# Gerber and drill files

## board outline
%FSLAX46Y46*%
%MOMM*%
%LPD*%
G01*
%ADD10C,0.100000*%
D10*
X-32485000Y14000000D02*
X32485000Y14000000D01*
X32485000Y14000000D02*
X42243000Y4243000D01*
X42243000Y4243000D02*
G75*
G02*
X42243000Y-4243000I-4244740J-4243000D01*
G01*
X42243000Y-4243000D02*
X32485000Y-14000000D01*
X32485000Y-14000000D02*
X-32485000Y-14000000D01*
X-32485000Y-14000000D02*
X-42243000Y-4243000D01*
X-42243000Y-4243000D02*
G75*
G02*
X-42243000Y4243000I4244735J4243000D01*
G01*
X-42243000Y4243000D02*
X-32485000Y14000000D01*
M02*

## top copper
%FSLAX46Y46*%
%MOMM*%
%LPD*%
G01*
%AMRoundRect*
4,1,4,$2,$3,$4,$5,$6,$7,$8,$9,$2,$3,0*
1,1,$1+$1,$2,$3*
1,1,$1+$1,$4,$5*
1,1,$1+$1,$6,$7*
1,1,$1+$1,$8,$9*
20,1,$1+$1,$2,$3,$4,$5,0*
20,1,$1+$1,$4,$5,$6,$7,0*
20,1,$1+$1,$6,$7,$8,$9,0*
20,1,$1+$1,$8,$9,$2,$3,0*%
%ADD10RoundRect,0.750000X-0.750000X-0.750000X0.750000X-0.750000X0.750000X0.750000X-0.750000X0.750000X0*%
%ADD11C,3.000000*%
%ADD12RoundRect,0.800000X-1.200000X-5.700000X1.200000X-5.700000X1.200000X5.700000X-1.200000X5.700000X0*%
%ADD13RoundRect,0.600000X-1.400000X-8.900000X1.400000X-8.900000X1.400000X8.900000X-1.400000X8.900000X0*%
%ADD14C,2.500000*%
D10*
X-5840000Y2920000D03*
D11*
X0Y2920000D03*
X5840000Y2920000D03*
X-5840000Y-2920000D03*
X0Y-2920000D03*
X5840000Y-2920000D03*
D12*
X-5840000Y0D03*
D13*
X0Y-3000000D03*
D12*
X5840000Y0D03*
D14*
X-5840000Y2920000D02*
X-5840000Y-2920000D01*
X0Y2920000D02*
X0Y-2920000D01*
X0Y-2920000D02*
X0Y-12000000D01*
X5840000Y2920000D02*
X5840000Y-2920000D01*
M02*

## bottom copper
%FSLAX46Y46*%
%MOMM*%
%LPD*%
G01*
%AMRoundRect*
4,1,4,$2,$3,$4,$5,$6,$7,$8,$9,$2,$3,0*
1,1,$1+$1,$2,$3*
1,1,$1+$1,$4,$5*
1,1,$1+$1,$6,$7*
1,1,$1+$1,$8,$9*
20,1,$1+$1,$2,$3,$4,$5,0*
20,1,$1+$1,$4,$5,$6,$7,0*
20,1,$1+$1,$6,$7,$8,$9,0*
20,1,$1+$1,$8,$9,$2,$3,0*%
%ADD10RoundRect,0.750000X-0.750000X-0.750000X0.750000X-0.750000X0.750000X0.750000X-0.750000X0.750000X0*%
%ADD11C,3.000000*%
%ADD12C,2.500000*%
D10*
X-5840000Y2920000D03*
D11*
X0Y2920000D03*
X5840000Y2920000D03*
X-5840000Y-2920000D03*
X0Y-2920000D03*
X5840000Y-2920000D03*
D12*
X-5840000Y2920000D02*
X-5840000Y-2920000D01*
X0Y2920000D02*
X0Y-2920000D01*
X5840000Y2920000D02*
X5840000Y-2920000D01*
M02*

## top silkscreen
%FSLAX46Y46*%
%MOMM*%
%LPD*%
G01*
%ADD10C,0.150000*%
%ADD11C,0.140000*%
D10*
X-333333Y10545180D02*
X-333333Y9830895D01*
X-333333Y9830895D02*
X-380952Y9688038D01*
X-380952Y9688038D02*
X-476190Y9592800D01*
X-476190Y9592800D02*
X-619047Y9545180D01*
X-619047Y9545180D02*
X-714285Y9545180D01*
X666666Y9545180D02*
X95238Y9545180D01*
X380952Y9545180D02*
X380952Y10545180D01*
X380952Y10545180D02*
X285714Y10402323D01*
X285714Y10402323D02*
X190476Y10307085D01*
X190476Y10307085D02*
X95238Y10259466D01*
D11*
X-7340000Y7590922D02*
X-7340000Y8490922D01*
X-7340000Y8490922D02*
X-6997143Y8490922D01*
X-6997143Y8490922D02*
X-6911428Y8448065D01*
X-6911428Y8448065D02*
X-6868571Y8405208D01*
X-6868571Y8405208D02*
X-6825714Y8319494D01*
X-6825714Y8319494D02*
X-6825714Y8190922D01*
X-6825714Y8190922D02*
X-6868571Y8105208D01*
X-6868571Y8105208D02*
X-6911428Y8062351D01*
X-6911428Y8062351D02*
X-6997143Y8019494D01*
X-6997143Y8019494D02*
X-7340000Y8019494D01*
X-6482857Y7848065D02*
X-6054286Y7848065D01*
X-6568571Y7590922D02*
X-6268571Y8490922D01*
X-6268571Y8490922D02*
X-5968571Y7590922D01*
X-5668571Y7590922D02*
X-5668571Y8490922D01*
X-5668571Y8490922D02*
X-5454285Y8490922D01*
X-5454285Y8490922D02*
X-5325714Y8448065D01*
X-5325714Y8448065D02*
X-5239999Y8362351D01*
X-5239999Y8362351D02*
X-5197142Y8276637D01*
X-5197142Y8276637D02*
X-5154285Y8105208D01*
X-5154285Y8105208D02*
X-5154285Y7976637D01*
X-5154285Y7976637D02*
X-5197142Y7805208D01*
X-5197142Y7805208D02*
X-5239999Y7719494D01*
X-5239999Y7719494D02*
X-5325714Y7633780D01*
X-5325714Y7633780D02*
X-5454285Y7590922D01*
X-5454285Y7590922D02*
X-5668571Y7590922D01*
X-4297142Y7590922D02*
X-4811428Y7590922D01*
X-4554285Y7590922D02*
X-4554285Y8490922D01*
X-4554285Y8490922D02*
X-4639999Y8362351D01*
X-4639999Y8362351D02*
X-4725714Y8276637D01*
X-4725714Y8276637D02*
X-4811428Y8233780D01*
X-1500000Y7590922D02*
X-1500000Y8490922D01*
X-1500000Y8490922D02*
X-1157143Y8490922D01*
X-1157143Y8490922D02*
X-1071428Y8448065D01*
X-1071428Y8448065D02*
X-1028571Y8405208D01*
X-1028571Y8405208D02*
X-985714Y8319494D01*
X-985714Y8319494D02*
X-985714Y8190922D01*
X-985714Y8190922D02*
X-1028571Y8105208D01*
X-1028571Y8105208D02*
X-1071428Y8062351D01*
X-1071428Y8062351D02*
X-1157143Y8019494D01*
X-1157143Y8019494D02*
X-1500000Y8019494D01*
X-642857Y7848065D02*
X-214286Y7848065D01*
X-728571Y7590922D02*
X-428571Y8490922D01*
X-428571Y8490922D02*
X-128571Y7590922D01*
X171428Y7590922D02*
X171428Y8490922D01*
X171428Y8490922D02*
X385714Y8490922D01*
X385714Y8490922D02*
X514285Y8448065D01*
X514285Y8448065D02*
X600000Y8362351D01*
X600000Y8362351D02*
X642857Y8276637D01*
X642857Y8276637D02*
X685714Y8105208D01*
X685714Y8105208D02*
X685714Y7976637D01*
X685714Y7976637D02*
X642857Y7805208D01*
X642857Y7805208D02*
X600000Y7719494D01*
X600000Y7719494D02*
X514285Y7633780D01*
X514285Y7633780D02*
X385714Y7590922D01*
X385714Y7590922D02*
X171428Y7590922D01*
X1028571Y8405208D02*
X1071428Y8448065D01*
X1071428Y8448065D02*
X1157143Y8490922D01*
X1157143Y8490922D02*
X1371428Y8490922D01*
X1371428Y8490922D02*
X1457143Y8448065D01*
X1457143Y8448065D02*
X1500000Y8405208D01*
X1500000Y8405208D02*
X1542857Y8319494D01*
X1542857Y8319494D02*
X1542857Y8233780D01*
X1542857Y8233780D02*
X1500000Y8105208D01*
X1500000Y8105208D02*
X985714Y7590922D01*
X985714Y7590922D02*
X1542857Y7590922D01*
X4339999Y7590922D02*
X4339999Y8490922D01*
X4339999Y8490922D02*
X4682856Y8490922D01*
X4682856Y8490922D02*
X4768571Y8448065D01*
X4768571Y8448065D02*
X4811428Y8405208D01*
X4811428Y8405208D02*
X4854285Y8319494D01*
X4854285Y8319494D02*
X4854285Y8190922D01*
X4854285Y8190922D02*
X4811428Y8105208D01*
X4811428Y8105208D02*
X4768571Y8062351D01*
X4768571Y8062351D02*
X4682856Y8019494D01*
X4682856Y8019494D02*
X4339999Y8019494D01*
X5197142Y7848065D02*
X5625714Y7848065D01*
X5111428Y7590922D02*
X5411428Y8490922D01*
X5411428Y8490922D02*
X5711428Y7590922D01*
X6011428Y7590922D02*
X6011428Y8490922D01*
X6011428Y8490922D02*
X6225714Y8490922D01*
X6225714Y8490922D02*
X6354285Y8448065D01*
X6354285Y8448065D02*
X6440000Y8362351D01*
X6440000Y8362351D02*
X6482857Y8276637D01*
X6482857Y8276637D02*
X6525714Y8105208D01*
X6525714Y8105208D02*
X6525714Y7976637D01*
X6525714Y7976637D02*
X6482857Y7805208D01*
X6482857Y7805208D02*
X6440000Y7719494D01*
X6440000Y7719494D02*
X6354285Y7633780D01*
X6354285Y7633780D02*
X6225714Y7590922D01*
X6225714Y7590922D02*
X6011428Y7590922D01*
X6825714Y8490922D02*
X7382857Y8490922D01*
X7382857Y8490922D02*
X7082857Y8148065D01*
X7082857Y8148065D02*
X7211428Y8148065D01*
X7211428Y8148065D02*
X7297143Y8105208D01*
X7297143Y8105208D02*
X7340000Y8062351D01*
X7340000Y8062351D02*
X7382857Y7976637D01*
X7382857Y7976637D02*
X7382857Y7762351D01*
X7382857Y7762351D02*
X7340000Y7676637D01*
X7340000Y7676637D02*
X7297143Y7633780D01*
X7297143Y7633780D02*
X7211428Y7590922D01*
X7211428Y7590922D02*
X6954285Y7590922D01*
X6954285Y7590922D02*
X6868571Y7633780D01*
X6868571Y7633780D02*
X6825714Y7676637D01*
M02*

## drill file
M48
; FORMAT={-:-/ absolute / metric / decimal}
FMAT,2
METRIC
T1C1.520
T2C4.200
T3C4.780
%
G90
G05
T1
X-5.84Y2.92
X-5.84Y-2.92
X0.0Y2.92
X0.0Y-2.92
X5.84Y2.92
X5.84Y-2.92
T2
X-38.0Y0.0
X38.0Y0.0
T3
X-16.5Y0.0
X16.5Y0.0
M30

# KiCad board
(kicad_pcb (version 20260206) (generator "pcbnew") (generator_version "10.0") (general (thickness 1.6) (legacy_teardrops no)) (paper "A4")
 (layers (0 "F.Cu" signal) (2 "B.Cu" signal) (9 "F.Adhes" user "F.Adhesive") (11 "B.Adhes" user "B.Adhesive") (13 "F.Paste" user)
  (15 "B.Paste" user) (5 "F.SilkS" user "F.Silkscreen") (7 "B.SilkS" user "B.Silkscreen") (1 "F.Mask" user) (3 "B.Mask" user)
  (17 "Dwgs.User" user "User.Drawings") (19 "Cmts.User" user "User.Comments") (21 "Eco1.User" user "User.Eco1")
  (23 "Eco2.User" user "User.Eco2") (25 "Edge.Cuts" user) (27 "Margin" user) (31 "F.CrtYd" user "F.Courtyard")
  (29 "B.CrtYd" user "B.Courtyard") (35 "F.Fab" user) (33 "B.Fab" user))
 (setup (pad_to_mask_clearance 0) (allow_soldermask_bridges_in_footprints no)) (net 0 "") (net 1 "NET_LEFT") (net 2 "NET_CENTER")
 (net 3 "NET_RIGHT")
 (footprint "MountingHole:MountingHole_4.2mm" (layer "F.Cu") (at -38 0)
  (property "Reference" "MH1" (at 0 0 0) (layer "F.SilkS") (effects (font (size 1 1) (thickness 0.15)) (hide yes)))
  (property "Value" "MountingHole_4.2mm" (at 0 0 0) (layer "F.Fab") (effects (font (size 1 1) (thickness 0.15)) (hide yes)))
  (pad "" np_thru_hole circle (at 0 0) (size 4.2 4.2) (drill 4.2) (layers "*.Mask")))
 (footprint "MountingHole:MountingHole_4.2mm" (layer "F.Cu") (at 38 0)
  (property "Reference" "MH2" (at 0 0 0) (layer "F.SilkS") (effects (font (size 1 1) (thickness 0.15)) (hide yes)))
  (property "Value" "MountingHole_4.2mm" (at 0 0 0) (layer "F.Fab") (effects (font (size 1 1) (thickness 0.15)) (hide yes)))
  (pad "" np_thru_hole circle (at 0 0) (size 4.2 4.2) (drill 4.2) (layers "*.Mask")))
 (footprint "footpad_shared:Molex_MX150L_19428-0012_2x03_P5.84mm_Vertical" (layer "F.Cu") (at 0 0)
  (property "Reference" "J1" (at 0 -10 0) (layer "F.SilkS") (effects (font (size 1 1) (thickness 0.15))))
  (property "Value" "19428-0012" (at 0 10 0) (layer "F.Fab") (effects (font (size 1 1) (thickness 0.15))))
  (pad "1" thru_hole roundrect (at -5.84 -2.92) (size 3 3) (drill 1.52) (layers "*.Cu" "*.Mask") (roundrect_rratio 0.25) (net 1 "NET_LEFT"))
  (pad "2" thru_hole circle (at 0 -2.92) (size 3 3) (drill 1.52) (layers "*.Cu" "*.Mask") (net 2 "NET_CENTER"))
  (pad "3" thru_hole circle (at 5.84 -2.92) (size 3 3) (drill 1.52) (layers "*.Cu" "*.Mask") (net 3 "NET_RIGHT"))
  (pad "4" thru_hole circle (at -5.84 2.92) (size 3 3) (drill 1.52) (layers "*.Cu" "*.Mask") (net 1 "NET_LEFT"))
  (pad "5" thru_hole circle (at 0 2.92) (size 3 3) (drill 1.52) (layers "*.Cu" "*.Mask") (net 2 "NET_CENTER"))
  (pad "6" thru_hole circle (at 5.84 2.92) (size 3 3) (drill 1.52) (layers "*.Cu" "*.Mask") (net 3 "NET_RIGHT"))
  (pad "MP1" np_thru_hole circle (at -16.5 0) (size 4.78 4.78) (drill 4.78) (layers "*.Cu" "*.Mask"))
  (pad "MP2" np_thru_hole circle (at 16.5 0) (size 4.78 4.78) (drill 4.78) (layers "*.Cu" "*.Mask")))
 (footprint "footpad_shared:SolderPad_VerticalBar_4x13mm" (layer "F.Cu") (at -5.84 0)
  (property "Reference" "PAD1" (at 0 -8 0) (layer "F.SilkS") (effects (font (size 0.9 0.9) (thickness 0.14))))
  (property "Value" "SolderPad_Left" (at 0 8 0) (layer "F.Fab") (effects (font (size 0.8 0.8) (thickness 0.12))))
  (pad "1" smd roundrect (at 0 0) (size 4 13) (layers "F.Cu" "F.Mask") (roundrect_rratio 0.2) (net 1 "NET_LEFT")))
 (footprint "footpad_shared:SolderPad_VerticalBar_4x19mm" (layer "F.Cu") (at 0 3)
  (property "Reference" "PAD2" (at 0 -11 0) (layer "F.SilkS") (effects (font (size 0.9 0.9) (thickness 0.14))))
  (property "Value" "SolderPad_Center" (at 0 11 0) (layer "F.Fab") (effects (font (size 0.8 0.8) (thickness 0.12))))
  (pad "1" smd roundrect (at 0 0) (size 4 19) (layers "F.Cu" "F.Mask") (roundrect_rratio 0.15) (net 2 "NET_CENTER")))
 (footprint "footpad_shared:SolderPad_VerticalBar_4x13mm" (layer "F.Cu") (at 5.84 0)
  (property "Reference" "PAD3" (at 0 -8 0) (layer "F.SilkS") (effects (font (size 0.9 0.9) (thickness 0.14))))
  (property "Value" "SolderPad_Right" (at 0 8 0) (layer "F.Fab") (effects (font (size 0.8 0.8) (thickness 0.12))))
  (pad "1" smd roundrect (at 0 0) (size 4 13) (layers "F.Cu" "F.Mask") (roundrect_rratio 0.2) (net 3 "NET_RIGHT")))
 (gr_line (start -32.485 -14) (end 32.485 -14) (stroke (width 0.1) (type default)) (layer "Edge.Cuts"))
 (gr_line (start 32.485 -14) (end 42.243 -4.243) (stroke (width 0.1) (type default)) (layer "Edge.Cuts"))
 (gr_arc (start 42.243 -4.243) (mid 44 0) (end 42.243 4.243) (stroke (width 0.1) (type default)) (layer "Edge.Cuts"))
 (gr_line (start 42.243 4.243) (end 32.485 14) (stroke (width 0.1) (type default)) (layer "Edge.Cuts"))
 (gr_line (start 32.485 14) (end -32.485 14) (stroke (width 0.1) (type default)) (layer "Edge.Cuts"))
 (gr_line (start -32.485 14) (end -42.243 4.243) (stroke (width 0.1) (type default)) (layer "Edge.Cuts"))
 (gr_arc (start -42.243 4.243) (mid -44 0) (end -42.243 -4.243) (stroke (width 0.1) (type default)) (layer "Edge.Cuts"))
 (gr_line (start -42.243 -4.243) (end -32.485 -14) (stroke (width 0.1) (type default)) (layer "Edge.Cuts"))
 (segment (start -5.84 -2.92) (end -5.84 2.92) (width 2.5) (layer "F.Cu") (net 1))
 (segment (start -5.84 -2.92) (end -5.84 2.92) (width 2.5) (layer "B.Cu") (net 1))
 (segment (start 0 -2.92) (end 0 2.92) (width 2.5) (layer "F.Cu") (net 2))
 (segment (start 0 -2.92) (end 0 2.92) (width 2.5) (layer "B.Cu") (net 2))
 (segment (start 0 2.92) (end 0 12.0) (width 2.5) (layer "F.Cu") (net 2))
 (segment (start 5.84 -2.92) (end 5.84 2.92) (width 2.5) (layer "F.Cu") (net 3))
 (segment (start 5.84 -2.92) (end 5.84 2.92) (width 2.5) (layer "B.Cu") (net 3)))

